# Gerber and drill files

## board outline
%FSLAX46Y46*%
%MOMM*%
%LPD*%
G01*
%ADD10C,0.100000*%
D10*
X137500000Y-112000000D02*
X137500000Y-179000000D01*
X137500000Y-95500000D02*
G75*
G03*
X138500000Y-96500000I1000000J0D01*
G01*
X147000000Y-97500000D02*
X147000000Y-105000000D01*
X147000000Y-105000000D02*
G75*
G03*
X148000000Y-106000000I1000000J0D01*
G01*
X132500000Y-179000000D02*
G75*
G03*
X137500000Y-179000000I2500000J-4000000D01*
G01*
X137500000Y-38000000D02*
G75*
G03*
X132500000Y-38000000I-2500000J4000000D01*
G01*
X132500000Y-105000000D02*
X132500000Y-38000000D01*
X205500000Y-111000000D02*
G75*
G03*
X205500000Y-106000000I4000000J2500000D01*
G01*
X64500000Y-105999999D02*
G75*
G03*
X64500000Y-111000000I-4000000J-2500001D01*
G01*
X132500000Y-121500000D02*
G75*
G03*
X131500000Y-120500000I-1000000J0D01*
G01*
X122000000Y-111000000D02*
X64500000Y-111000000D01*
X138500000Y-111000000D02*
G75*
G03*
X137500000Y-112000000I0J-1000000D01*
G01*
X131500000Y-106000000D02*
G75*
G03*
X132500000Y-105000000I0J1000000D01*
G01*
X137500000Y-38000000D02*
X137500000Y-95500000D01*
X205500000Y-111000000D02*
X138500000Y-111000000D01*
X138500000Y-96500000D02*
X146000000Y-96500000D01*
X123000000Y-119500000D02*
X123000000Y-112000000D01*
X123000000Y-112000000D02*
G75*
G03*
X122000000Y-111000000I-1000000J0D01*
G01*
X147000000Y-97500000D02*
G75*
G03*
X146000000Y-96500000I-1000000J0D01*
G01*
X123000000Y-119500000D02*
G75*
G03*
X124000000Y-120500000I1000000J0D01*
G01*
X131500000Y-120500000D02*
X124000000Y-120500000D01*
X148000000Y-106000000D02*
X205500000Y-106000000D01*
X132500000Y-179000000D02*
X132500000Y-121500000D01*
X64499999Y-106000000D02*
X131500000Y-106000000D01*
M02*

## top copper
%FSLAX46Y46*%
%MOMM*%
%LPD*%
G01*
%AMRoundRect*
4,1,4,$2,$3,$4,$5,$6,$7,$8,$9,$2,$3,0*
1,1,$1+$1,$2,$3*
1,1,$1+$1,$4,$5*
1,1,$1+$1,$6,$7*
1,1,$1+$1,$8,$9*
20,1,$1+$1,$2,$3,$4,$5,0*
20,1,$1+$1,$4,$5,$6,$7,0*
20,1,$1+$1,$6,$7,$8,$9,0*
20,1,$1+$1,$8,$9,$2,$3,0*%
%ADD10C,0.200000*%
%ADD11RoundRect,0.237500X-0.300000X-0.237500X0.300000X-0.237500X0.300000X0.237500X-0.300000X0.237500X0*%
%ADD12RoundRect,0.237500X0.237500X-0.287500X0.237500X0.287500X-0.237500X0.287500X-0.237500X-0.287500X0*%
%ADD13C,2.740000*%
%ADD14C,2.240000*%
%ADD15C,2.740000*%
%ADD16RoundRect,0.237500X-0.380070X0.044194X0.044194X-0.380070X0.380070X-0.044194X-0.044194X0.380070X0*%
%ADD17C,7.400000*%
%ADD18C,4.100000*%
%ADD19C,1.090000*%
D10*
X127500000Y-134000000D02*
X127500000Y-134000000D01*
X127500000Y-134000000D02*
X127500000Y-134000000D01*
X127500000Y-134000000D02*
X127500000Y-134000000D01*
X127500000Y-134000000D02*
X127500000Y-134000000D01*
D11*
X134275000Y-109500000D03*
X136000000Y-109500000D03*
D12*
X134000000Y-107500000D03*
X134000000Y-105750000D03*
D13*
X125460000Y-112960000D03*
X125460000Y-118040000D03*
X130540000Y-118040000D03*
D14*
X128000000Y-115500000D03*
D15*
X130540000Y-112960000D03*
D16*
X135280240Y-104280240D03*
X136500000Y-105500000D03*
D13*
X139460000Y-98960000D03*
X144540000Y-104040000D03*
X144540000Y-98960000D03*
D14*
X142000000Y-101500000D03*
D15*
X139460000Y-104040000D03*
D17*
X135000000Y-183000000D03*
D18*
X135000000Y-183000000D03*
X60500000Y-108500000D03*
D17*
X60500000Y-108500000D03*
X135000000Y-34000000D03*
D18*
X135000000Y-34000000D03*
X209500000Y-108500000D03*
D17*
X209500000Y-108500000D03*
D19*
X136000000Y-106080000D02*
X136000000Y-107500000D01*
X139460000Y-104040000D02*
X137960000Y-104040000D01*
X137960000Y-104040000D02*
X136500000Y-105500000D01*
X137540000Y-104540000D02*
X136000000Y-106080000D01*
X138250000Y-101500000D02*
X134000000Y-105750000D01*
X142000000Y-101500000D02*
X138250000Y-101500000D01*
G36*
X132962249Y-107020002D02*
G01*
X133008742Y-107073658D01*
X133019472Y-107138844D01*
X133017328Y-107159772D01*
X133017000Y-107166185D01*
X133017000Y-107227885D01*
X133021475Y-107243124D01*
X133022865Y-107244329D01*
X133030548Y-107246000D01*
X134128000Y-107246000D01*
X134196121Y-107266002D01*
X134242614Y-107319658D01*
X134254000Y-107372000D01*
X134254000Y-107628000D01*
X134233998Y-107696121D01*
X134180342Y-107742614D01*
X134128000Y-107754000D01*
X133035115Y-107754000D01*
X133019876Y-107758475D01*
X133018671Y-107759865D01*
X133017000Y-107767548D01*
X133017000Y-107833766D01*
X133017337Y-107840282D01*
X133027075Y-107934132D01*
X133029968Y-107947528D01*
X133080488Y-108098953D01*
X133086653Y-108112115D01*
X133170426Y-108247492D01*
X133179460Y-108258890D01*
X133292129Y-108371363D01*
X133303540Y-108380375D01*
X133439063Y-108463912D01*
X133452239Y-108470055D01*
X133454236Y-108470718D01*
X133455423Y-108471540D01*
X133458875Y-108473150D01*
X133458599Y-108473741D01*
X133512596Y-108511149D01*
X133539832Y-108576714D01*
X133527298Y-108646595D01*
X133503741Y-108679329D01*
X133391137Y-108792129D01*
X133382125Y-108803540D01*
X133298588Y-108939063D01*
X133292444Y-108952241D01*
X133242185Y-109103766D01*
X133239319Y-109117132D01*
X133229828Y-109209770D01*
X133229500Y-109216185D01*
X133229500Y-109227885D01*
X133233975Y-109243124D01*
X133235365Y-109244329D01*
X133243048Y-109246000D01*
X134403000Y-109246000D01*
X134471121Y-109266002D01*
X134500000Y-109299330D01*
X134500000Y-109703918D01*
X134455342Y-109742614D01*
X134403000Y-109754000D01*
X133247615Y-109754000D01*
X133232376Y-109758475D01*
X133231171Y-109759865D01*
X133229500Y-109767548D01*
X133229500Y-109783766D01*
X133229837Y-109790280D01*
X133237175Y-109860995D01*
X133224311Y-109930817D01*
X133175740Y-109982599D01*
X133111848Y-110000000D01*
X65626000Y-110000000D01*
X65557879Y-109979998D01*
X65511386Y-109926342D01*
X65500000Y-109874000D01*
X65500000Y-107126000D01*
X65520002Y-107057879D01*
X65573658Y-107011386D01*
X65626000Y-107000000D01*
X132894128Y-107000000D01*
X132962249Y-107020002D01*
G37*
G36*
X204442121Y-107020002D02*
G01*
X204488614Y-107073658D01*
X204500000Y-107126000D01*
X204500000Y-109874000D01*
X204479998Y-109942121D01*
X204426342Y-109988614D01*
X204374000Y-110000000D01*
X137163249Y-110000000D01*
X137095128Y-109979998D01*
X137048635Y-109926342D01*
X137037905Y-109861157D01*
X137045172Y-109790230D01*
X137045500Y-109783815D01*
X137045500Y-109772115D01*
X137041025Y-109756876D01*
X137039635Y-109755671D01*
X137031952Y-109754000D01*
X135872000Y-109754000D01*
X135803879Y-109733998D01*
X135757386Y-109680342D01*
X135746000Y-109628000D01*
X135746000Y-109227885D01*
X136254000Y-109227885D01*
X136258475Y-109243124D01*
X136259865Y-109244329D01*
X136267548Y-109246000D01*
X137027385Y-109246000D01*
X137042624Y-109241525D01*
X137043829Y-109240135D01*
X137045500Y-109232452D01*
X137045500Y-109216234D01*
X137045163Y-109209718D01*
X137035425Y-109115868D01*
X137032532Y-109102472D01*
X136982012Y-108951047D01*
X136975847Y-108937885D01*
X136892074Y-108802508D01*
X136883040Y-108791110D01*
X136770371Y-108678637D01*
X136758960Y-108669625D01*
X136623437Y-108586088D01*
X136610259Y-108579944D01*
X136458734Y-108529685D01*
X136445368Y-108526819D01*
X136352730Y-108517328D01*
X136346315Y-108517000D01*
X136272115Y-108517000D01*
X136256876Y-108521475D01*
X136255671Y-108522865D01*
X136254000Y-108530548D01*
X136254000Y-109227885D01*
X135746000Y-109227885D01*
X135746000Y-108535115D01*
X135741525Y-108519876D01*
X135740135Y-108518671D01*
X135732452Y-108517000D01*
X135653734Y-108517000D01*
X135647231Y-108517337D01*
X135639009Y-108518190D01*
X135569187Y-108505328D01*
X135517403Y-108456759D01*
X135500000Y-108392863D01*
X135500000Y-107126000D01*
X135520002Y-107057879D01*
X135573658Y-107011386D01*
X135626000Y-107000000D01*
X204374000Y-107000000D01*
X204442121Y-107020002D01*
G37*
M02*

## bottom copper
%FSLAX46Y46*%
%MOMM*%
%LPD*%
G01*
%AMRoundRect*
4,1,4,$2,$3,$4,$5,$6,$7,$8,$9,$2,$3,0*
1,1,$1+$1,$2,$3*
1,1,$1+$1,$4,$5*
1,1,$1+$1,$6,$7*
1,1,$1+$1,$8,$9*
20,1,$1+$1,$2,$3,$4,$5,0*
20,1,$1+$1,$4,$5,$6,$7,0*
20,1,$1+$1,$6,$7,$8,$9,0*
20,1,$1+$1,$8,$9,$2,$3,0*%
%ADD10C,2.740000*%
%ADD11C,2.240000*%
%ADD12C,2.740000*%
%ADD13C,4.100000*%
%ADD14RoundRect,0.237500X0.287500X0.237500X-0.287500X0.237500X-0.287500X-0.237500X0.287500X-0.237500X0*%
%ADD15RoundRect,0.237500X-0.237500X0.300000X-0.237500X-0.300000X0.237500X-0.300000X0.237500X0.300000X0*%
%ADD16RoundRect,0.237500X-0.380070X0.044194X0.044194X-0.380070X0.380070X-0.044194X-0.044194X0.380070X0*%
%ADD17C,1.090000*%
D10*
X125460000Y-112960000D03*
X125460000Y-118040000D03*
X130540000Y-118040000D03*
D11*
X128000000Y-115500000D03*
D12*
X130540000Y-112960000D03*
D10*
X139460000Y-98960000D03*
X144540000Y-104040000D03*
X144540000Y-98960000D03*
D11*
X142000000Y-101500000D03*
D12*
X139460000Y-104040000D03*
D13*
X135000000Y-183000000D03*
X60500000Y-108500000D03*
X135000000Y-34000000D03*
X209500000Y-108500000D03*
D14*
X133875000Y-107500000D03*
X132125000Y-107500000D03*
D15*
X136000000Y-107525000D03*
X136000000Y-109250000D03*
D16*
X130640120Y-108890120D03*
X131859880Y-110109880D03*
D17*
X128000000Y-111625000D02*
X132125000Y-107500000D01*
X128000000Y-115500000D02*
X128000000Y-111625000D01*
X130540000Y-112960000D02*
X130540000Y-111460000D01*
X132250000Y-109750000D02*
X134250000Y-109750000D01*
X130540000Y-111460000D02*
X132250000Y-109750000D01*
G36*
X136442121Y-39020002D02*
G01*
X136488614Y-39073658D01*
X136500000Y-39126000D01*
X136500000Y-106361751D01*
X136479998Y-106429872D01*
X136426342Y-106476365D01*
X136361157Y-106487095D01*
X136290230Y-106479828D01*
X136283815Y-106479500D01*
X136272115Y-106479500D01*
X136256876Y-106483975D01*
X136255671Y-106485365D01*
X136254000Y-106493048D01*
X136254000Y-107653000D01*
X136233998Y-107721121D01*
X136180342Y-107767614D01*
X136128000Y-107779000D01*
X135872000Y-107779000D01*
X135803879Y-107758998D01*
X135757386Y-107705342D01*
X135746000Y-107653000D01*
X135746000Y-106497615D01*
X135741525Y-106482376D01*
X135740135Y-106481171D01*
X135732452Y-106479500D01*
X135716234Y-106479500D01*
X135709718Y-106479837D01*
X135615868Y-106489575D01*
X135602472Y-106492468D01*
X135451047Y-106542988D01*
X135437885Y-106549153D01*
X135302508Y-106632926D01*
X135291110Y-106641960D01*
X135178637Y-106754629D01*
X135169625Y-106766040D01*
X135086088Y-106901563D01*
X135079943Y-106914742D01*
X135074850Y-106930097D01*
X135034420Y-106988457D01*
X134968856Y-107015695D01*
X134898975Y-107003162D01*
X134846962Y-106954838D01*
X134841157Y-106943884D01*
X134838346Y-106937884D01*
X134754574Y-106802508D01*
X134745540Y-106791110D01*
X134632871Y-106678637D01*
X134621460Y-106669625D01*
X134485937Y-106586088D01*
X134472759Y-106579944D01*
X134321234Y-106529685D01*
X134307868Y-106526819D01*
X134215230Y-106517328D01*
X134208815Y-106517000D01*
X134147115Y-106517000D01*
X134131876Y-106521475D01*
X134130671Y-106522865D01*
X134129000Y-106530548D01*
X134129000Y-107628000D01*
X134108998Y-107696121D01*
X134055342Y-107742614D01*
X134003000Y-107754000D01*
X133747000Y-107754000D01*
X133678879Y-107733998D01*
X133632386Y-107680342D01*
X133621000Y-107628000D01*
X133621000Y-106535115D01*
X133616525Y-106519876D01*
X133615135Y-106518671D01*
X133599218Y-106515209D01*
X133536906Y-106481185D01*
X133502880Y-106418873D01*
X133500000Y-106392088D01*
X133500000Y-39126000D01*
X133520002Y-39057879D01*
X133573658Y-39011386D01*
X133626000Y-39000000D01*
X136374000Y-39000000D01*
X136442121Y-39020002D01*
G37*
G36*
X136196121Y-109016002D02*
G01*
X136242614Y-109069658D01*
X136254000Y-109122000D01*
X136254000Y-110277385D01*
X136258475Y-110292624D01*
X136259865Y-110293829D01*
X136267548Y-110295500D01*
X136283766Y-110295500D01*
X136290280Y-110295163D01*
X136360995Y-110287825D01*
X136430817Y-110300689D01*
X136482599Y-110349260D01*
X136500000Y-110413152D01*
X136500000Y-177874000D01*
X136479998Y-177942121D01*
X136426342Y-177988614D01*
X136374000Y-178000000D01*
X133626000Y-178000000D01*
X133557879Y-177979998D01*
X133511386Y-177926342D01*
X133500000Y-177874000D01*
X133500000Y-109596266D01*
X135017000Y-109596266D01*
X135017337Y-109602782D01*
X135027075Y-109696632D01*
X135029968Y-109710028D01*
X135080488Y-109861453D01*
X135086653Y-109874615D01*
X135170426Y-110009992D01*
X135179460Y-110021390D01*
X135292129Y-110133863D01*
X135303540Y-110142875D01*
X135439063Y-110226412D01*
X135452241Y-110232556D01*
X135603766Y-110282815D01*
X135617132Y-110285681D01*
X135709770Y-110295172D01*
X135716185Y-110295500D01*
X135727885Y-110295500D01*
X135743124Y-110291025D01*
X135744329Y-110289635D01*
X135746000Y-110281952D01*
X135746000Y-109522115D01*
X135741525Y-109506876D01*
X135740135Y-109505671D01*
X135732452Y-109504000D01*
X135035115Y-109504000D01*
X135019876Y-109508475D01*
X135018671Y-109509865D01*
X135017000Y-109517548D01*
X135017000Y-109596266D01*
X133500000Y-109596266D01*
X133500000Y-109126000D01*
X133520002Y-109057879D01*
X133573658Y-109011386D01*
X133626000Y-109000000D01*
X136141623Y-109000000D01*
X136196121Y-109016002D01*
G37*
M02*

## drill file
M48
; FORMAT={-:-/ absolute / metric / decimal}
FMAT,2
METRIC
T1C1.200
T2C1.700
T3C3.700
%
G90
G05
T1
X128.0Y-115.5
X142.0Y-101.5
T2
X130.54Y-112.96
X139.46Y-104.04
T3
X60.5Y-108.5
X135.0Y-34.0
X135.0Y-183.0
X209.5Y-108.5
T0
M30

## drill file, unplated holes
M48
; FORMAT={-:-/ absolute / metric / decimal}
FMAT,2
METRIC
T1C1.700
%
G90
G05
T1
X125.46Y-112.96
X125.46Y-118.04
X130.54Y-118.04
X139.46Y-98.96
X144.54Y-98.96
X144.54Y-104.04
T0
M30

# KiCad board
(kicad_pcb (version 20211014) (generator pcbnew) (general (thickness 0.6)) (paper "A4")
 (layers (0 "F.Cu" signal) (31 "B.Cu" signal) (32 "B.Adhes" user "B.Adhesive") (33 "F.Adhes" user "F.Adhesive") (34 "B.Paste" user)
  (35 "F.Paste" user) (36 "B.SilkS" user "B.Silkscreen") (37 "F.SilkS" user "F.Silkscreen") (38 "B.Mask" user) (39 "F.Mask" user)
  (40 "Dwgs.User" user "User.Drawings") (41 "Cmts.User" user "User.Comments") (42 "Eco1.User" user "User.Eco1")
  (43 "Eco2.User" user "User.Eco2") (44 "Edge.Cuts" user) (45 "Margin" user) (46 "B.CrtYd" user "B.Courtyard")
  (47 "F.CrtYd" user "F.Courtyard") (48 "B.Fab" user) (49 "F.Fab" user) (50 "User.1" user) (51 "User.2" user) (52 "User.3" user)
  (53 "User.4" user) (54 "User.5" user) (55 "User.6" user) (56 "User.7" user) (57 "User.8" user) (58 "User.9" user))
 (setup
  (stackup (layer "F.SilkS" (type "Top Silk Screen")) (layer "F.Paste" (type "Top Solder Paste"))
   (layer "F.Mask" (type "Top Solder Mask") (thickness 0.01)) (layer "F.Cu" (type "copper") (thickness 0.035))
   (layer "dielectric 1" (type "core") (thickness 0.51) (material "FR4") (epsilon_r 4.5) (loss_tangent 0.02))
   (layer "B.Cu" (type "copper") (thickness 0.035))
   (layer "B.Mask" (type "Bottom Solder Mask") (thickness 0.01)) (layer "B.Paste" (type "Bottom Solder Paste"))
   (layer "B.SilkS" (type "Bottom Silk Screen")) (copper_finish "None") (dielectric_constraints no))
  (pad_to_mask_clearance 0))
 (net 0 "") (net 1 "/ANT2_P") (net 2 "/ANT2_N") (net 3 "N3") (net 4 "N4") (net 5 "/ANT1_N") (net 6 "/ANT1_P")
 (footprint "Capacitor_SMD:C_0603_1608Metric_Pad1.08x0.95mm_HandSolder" (layer "F.Cu") (at 135.1375 109.5)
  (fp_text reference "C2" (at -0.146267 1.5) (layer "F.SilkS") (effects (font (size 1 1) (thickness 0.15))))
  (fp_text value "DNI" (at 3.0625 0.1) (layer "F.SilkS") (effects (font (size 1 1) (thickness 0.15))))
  (pad "1" smd roundrect (at -0.8625 0) (size 1.075 0.95) (layers "F.Cu" "F.Paste" "F.Mask") (roundrect_rratio 0.25) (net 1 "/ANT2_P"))
  (pad "2" smd roundrect (at 0.8625 0) (size 1.075 0.95) (layers "F.Cu" "F.Paste" "F.Mask") (roundrect_rratio 0.25) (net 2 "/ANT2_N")))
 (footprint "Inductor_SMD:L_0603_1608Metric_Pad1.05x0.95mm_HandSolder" (layer "F.Cu") (at 134 106.625 90)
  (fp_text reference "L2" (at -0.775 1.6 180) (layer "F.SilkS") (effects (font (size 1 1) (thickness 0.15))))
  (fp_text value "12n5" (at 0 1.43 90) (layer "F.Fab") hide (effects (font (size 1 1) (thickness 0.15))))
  (pad "1" smd roundrect (at -0.875 0 90) (size 1.05 0.95) (layers "F.Cu" "F.Paste" "F.Mask") (roundrect_rratio 0.25) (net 1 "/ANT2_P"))
  (pad "2" smd roundrect (at 0.875 0 90) (size 1.05 0.95) (layers "F.Cu" "F.Paste" "F.Mask") (roundrect_rratio 0.25) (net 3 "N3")))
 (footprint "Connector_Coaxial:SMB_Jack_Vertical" (layer "F.Cu") (at 128 115.5)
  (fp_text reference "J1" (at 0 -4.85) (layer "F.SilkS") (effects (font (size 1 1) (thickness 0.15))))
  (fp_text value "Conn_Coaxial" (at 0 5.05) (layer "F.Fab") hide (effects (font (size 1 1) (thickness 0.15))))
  (pad "" np_thru_hole circle (at -2.54 -2.54) (size 2.74 2.74) (drill 1.7) (layers F&B.Cu *.Mask))
  (pad "" np_thru_hole circle (at -2.54 2.54) (size 2.74 2.74) (drill 1.7) (layers F&B.Cu *.Mask))
  (pad "" np_thru_hole circle (at 2.54 2.54) (size 2.74 2.74) (drill 1.7) (layers F&B.Cu *.Mask))
  (pad "1" thru_hole circle (at 0 0) (size 2.24 2.24) (drill 1.2) (layers *.Cu *.Mask) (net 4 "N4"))
  (pad "2" thru_hole circle (at 2.54 -2.54) (size 2.74 2.74) (drill 1.7) (layers *.Cu *.Mask) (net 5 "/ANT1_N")))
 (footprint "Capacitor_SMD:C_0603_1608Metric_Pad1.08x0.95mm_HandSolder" (layer "F.Cu") (at 135.89012 104.89012 -45)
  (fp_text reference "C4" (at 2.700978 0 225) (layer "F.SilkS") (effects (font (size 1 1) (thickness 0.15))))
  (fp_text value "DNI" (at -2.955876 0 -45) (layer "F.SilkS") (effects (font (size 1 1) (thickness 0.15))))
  (pad "1" smd roundrect (at -0.8625 0 315) (size 1.075 0.95) (layers "F.Cu" "F.Paste" "F.Mask") (roundrect_rratio 0.25) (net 3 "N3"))
  (pad "2" smd roundrect (at 0.8625 0 315) (size 1.075 0.95) (layers "F.Cu" "F.Paste" "F.Mask") (roundrect_rratio 0.25) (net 2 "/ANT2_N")))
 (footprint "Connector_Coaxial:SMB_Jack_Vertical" (layer "F.Cu") (at 142 101.5)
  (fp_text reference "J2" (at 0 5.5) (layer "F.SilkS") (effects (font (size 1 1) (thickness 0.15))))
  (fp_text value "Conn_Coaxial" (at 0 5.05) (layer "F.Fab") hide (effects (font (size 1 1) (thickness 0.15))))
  (pad "" np_thru_hole circle (at -2.54 -2.54) (size 2.74 2.74) (drill 1.7) (layers F&B.Cu *.Mask))
  (pad "" np_thru_hole circle (at 2.54 2.54) (size 2.74 2.74) (drill 1.7) (layers F&B.Cu *.Mask))
  (pad "" np_thru_hole circle (at 2.54 -2.54) (size 2.74 2.74) (drill 1.7) (layers F&B.Cu *.Mask))
  (pad "1" thru_hole circle (at 0 0) (size 2.24 2.24) (drill 1.2) (layers *.Cu *.Mask) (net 3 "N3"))
  (pad "2" thru_hole circle (at -2.54 2.54) (size 2.74 2.74) (drill 1.7) (layers *.Cu *.Mask) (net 2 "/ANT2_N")))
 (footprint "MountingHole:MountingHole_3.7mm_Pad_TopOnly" (layer "F.Cu") (at 135 183)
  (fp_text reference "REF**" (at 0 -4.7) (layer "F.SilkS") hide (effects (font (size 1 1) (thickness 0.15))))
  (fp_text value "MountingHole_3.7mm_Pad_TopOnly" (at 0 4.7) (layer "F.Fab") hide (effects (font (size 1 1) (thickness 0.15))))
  (pad "1" connect circle (at 0 0) (size 7.4 7.4) (layers "F.Cu" "F.Mask"))
  (pad "1" thru_hole circle (at 0 0) (size 4.1 4.1) (drill 3.7) (layers *.Cu *.Mask)))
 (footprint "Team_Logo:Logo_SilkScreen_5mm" (layer "F.Cu") (at 135.2 97.2)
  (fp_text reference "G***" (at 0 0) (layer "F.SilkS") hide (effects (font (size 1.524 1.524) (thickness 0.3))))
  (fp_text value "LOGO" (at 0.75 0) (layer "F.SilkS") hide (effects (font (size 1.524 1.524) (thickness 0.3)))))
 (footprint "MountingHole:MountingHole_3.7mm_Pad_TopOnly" (layer "F.Cu") (at 60.5 108.5)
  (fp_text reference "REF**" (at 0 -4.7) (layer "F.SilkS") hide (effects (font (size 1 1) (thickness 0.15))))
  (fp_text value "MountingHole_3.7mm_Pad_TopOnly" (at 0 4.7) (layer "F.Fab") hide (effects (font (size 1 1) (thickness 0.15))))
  (pad "1" thru_hole circle (at 0 0) (size 4.1 4.1) (drill 3.7) (layers *.Cu *.Mask))
  (pad "1" connect circle (at 0 0) (size 7.4 7.4) (layers "F.Cu" "F.Mask")))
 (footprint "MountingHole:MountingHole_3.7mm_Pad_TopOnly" (layer "F.Cu") (at 135 34)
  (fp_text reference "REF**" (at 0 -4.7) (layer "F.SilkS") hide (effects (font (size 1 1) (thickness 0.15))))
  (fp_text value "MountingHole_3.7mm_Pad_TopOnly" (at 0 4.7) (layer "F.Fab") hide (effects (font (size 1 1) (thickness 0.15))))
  (pad "1" connect circle (at 0 0) (size 7.4 7.4) (layers "F.Cu" "F.Mask"))
  (pad "1" thru_hole circle (at 0 0) (size 4.1 4.1) (drill 3.7) (layers *.Cu *.Mask)))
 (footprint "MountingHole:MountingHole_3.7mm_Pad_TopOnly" (layer "F.Cu") (at 209.5 108.5)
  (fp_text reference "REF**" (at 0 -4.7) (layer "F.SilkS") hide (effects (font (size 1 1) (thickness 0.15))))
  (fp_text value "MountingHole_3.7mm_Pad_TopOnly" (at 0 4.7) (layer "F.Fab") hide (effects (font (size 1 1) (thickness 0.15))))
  (pad "1" thru_hole circle (at 0 0) (size 4.1 4.1) (drill 3.7) (layers *.Cu *.Mask))
  (pad "1" connect circle (at 0 0) (size 7.4 7.4) (layers "F.Cu" "F.Mask")))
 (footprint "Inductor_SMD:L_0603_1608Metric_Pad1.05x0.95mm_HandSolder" (layer "B.Cu") (at 133 107.5 180)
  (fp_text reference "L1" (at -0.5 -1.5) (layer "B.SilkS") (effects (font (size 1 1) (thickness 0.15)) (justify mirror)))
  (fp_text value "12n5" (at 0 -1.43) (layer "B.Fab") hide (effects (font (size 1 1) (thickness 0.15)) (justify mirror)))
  (pad "1" smd roundrect (at -0.875 0 180) (size 1.05 0.95) (layers "B.Cu" "B.Paste" "B.Mask") (roundrect_rratio 0.25) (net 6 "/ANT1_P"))
  (pad "2" smd roundrect (at 0.875 0 180) (size 1.05 0.95) (layers "B.Cu" "B.Paste" "B.Mask") (roundrect_rratio 0.25) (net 4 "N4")))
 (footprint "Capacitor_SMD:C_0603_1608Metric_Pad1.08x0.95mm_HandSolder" (layer "B.Cu") (at 136 108.3875 -90)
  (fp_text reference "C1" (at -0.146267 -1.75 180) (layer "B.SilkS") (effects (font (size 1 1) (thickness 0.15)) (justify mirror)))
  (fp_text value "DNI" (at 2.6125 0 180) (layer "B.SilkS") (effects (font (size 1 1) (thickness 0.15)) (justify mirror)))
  (pad "1" smd roundrect (at -0.8625 0 270) (size 1.075 0.95) (layers "B.Cu" "B.Paste" "B.Mask") (roundrect_rratio 0.25) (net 6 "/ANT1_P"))
  (pad "2" smd roundrect (at 0.8625 0 270) (size 1.075 0.95) (layers "B.Cu" "B.Paste" "B.Mask") (roundrect_rratio 0.25) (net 5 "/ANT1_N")))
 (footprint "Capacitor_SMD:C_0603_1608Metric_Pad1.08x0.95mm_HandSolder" (layer "B.Cu") (at 131.25 109.5 -45)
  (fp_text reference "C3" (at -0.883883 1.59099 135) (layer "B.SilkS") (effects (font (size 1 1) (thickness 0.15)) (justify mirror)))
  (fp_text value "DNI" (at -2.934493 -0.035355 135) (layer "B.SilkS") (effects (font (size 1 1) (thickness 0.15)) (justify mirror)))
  (pad "1" smd roundrect (at -0.8625 0 315) (size 1.075 0.95) (layers "B.Cu" "B.Paste" "B.Mask") (roundrect_rratio 0.25) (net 4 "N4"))
  (pad "2" smd roundrect (at 0.8625 0 315) (size 1.075 0.95) (layers "B.Cu" "B.Paste" "B.Mask") (roundrect_rratio 0.25) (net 5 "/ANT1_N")))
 (gr_rect (start 127.5 134) (end 127.5 134) (layer "F.Cu") (width 0.2) (fill none))
 (gr_line (start 137.5 112) (end 137.5 179) (layer "Edge.Cuts") (width 0.1))
 (gr_arc (start 138.5 96.5) (mid 137.792893 96.207107) (end 137.5 95.5) (layer "Edge.Cuts") (width 0.1))
 (gr_line (start 147 97.5) (end 147 105) (layer "Edge.Cuts") (width 0.1))
 (gr_arc (start 148 106) (mid 147.292893 105.707107) (end 147 105) (layer "Edge.Cuts") (width 0.1))
 (gr_arc (start 137.5 179) (mid 135 187.716991) (end 132.5 179) (layer "Edge.Cuts") (width 0.1))
 (gr_arc (start 132.5 38) (mid 135 29.283009) (end 137.5 38) (layer "Edge.Cuts") (width 0.1))
 (gr_line (start 132.5 105) (end 132.5 38) (layer "Edge.Cuts") (width 0.1))
 (gr_arc (start 205.5 106) (mid 214.216991 108.5) (end 205.5 111) (layer "Edge.Cuts") (width 0.1))
 (gr_arc (start 64.5 111) (mid 55.783009 108.5) (end 64.499999 106) (layer "Edge.Cuts") (width 0.1))
 (gr_arc (start 131.5 120.5) (mid 132.207107 120.792893) (end 132.5 121.5) (layer "Edge.Cuts") (width 0.1))
 (gr_line (start 122 111) (end 64.5 111) (layer "Edge.Cuts") (width 0.1))
 (gr_arc (start 137.5 112) (mid 137.792893 111.292893) (end 138.5 111) (layer "Edge.Cuts") (width 0.1))
 (gr_arc (start 132.5 105) (mid 132.207107 105.707107) (end 131.5 106) (layer "Edge.Cuts") (width 0.1))
 (gr_line (start 137.5 38) (end 137.5 95.5) (layer "Edge.Cuts") (width 0.1))
 (gr_line (start 205.5 111) (end 138.5 111) (layer "Edge.Cuts") (width 0.1))
 (gr_line (start 138.5 96.5) (end 146 96.5) (layer "Edge.Cuts") (width 0.1))
 (gr_line (start 123 119.5) (end 123 112) (layer "Edge.Cuts") (width 0.1))
 (gr_arc (start 122 111) (mid 122.707107 111.292893) (end 123 112) (layer "Edge.Cuts") (width 0.1))
 (gr_arc (start 146 96.5) (mid 146.707107 96.792893) (end 147 97.5) (layer "Edge.Cuts") (width 0.1))
 (gr_arc (start 124 120.5) (mid 123.292893 120.207107) (end 123 119.5) (layer "Edge.Cuts") (width 0.1))
 (gr_line (start 131.5 120.5) (end 124 120.5) (layer "Edge.Cuts") (width 0.1))
 (gr_line (start 148 106) (end 205.5 106) (layer "Edge.Cuts") (width 0.1))
 (gr_line (start 132.5 179) (end 132.5 121.5) (layer "Edge.Cuts") (width 0.1))
 (gr_line (start 64.499999 106) (end 131.5 106) (layer "Edge.Cuts") (width 0.1))
 (segment (start 128 111.625) (end 132.125 107.5) (width 1.09) (layer "B.Cu") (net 4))
 (segment (start 128 115.5) (end 128 111.625) (width 1.09) (layer "B.Cu") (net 4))
 (segment (start 130.54 112.96) (end 130.54 111.46) (width 1.09) (layer "B.Cu") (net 5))
 (segment (start 132.25 109.75) (end 134.25 109.75) (width 1.09) (layer "B.Cu") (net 5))
 (segment (start 130.54 111.46) (end 132.25 109.75) (width 1.09) (layer "B.Cu") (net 5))
 (segment (start 136 106.08) (end 136 107.5) (width 1.09) (layer "F.Cu") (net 2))
 (segment (start 139.46 104.04) (end 137.96 104.04) (width 1.09) (layer "F.Cu") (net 2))
 (segment (start 137.96 104.04) (end 136.5 105.5) (width 1.09) (layer "F.Cu") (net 2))
 (segment (start 137.54 104.54) (end 136 106.08) (width 1.09) (layer "F.Cu") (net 2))
 (segment (start 138.25 101.5) (end 134 105.75) (width 1.09) (layer "F.Cu") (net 3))
 (segment (start 142 101.5) (end 138.25 101.5) (width 1.09) (layer "F.Cu") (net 3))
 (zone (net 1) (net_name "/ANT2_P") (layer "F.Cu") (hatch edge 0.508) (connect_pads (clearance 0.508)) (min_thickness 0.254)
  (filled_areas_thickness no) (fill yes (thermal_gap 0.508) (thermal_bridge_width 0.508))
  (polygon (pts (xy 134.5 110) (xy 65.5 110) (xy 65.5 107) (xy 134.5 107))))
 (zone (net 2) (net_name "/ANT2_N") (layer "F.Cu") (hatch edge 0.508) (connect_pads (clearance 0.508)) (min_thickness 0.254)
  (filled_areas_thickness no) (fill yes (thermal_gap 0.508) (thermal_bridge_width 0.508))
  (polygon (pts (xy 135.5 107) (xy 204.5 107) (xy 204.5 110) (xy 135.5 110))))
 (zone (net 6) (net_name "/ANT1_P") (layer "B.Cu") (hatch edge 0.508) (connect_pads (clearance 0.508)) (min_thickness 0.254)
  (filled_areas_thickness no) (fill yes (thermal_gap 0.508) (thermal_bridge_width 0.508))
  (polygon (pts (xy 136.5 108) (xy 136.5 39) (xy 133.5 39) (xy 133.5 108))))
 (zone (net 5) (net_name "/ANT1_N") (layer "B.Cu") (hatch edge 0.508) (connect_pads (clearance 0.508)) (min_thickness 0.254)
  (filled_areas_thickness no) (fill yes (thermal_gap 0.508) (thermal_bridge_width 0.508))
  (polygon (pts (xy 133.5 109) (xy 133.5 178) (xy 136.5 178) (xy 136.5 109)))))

